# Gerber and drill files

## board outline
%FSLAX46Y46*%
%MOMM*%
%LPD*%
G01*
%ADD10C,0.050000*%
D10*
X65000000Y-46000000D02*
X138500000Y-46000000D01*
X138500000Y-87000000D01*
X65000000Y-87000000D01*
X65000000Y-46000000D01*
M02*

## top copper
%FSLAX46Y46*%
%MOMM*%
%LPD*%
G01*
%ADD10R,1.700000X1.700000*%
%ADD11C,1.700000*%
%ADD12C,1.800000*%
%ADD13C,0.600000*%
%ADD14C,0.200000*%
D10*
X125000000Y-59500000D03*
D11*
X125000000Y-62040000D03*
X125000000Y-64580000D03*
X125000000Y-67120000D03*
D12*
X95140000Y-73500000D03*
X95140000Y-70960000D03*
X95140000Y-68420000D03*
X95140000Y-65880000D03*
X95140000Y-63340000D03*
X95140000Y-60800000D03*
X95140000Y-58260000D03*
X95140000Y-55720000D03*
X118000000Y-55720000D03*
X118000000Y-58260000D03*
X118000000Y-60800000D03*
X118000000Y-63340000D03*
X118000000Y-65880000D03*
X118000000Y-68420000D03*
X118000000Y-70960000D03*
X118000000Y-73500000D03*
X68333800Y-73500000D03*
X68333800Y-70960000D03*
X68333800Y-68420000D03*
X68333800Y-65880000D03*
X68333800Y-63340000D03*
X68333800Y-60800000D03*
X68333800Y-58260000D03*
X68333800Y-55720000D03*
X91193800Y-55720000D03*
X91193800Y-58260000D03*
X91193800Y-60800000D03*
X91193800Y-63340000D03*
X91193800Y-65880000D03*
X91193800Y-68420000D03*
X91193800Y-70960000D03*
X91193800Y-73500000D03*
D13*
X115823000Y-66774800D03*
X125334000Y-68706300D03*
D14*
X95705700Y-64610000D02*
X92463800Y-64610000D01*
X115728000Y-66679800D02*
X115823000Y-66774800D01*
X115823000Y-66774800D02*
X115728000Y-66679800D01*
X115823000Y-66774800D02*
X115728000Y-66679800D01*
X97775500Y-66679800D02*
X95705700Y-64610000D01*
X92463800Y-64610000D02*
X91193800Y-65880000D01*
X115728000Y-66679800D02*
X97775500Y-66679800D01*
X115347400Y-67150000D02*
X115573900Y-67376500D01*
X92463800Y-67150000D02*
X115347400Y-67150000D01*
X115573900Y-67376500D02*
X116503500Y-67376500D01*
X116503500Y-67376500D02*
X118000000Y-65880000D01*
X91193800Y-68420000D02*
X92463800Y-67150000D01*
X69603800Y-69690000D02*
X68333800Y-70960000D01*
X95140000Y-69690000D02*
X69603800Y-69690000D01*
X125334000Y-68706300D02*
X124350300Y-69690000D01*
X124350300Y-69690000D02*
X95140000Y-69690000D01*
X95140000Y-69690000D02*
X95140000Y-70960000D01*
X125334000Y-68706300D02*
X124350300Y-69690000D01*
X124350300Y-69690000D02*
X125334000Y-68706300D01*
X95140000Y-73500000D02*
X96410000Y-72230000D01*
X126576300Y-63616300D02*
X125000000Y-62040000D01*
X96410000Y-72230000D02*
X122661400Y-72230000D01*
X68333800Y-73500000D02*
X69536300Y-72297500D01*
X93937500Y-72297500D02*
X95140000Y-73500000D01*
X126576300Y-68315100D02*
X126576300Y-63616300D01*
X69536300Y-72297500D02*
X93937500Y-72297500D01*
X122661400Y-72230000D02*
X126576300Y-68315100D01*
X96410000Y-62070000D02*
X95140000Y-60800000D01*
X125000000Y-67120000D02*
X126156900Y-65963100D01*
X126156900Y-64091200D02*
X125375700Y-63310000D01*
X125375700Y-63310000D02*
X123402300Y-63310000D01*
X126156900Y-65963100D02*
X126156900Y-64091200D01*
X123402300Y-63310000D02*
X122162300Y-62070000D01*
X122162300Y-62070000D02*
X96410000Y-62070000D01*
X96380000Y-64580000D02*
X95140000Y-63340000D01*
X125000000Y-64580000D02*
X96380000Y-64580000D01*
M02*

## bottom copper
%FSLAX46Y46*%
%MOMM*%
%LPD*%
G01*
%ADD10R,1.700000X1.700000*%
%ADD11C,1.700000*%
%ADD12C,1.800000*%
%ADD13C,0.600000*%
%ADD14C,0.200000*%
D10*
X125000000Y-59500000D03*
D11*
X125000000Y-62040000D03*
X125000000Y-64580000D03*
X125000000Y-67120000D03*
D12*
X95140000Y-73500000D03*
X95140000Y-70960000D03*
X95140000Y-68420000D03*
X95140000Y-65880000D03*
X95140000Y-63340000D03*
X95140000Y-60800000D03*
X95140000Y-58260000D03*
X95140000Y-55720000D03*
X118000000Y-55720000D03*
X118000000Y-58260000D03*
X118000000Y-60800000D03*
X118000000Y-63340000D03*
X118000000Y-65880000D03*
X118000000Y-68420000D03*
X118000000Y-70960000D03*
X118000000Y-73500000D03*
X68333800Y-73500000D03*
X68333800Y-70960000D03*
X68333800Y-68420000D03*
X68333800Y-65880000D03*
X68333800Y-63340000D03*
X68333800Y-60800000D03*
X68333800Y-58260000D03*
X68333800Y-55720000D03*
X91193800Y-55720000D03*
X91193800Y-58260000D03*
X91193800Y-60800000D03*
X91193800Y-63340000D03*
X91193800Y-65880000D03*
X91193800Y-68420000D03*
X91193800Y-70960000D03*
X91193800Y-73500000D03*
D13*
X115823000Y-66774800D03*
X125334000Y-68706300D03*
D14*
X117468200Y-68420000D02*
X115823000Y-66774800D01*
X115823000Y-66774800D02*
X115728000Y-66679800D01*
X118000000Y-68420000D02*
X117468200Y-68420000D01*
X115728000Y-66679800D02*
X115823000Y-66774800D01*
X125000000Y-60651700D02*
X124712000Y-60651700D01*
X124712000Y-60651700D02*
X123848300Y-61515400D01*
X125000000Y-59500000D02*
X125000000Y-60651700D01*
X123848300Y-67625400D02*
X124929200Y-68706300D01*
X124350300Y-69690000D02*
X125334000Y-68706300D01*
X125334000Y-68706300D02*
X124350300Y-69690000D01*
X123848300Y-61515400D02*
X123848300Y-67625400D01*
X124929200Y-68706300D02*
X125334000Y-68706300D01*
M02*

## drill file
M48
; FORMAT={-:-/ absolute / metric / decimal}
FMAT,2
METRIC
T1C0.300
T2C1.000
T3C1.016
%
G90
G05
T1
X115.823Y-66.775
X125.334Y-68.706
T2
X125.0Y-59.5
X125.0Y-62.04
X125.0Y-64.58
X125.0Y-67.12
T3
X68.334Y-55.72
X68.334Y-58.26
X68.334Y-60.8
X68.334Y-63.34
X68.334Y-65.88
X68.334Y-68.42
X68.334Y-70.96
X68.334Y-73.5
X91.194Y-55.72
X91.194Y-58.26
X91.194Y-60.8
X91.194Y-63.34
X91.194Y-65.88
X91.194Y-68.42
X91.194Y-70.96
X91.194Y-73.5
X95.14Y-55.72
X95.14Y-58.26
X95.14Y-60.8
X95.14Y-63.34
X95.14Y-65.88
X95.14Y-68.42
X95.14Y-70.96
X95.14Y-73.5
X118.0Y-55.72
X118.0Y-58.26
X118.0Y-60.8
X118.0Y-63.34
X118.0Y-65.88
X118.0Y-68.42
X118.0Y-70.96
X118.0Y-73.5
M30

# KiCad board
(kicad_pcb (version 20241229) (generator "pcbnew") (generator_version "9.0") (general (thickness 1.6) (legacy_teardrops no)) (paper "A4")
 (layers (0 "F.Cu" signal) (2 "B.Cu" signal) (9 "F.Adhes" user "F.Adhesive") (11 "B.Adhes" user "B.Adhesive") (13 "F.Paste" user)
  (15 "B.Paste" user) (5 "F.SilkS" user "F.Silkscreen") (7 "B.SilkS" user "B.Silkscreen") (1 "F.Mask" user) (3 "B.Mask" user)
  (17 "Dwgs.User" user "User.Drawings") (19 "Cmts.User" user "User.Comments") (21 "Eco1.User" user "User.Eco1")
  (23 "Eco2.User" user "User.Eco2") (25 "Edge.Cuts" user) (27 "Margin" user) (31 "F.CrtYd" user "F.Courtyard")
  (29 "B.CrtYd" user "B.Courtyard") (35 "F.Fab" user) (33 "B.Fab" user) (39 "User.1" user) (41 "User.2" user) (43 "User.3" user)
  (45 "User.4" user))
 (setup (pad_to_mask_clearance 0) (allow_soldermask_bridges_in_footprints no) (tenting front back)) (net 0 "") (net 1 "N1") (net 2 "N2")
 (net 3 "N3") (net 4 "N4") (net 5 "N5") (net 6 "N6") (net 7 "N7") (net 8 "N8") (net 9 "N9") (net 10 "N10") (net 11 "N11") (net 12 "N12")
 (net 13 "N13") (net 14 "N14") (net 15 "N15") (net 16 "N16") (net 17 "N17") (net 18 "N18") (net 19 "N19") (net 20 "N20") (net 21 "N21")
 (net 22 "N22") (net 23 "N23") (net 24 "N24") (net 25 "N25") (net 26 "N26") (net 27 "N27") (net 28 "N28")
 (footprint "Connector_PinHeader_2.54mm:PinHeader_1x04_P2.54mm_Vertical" (layer "F.Cu") (at 125 59.5)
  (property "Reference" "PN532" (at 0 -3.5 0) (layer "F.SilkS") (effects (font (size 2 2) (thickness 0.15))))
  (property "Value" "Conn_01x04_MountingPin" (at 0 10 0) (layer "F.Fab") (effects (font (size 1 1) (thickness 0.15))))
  (pad "1" thru_hole rect (at 0 0) (size 1.7 1.7) (drill 1) (layers "*.Cu" "*.Mask") (remove_unused_layers no) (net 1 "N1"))
  (pad "2" thru_hole circle (at 0 2.54) (size 1.7 1.7) (drill 1) (layers "*.Cu" "*.Mask") (remove_unused_layers no) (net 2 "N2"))
  (pad "3" thru_hole circle (at 0 5.08) (size 1.7 1.7) (drill 1) (layers "*.Cu" "*.Mask") (remove_unused_layers no) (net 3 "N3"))
  (pad "4" thru_hole circle (at 0 7.62) (size 1.7 1.7) (drill 1) (layers "*.Cu" "*.Mask") (remove_unused_layers no) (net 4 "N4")))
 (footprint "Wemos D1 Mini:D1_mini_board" (layer "F.Cu") (at 106.57 65.88)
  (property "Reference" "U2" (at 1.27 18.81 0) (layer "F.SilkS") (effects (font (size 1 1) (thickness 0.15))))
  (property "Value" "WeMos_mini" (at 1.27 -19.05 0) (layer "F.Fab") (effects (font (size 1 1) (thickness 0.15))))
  (pad "1" thru_hole circle (at -11.43 7.62) (size 1.8 1.8) (drill 1.016) (layers "*.Cu" "*.Mask" "F.SilkS") (remove_unused_layers no)
   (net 2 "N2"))
  (pad "2" thru_hole circle (at -11.43 5.08) (size 1.8 1.8) (drill 1.016) (layers "*.Cu" "*.Mask" "F.SilkS") (remove_unused_layers no)
   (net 1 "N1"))
  (pad "3" thru_hole circle (at -11.43 2.54) (size 1.8 1.8) (drill 1.016) (layers "*.Cu" "*.Mask" "F.SilkS") (remove_unused_layers no)
   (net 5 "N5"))
  (pad "4" thru_hole circle (at -11.43 0) (size 1.8 1.8) (drill 1.016) (layers "*.Cu" "*.Mask" "F.SilkS") (remove_unused_layers no)
   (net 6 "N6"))
  (pad "5" thru_hole circle (at -11.43 -2.54) (size 1.8 1.8) (drill 1.016) (layers "*.Cu" "*.Mask" "F.SilkS") (remove_unused_layers no)
   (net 3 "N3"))
  (pad "6" thru_hole circle (at -11.43 -5.08) (size 1.8 1.8) (drill 1.016) (layers "*.Cu" "*.Mask" "F.SilkS") (remove_unused_layers no)
   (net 4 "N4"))
  (pad "7" thru_hole circle (at -11.43 -7.62) (size 1.8 1.8) (drill 1.016) (layers "*.Cu" "*.Mask" "F.SilkS") (remove_unused_layers no)
   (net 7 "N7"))
  (pad "8" thru_hole circle (at -11.43 -10.16) (size 1.8 1.8) (drill 1.016) (layers "*.Cu" "*.Mask" "F.SilkS") (remove_unused_layers no)
   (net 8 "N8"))
  (pad "9" thru_hole circle (at 11.43 -10.16) (size 1.8 1.8) (drill 1.016) (layers "*.Cu" "*.Mask" "F.SilkS") (remove_unused_layers no)
   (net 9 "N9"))
  (pad "10" thru_hole circle (at 11.43 -7.62) (size 1.8 1.8) (drill 1.016) (layers "*.Cu" "*.Mask" "F.SilkS") (remove_unused_layers no)
   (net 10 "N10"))
  (pad "11" thru_hole circle (at 11.43 -5.08) (size 1.8 1.8) (drill 1.016) (layers "*.Cu" "*.Mask" "F.SilkS") (remove_unused_layers no)
   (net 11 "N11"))
  (pad "12" thru_hole circle (at 11.43 -2.54) (size 1.8 1.8) (drill 1.016) (layers "*.Cu" "*.Mask" "F.SilkS") (remove_unused_layers no)
   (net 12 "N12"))
  (pad "13" thru_hole circle (at 11.43 0) (size 1.8 1.8) (drill 1.016) (layers "*.Cu" "*.Mask" "F.SilkS") (remove_unused_layers no)
   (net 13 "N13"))
  (pad "14" thru_hole circle (at 11.43 2.54) (size 1.8 1.8) (drill 1.016) (layers "*.Cu" "*.Mask" "F.SilkS") (remove_unused_layers no)
   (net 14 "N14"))
  (pad "15" thru_hole circle (at 11.43 5.08) (size 1.8 1.8) (drill 1.016) (layers "*.Cu" "*.Mask" "F.SilkS") (remove_unused_layers no)
   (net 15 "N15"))
  (pad "16" thru_hole circle (at 11.43 7.62) (size 1.8 1.8) (drill 1.016) (layers "*.Cu" "*.Mask" "F.SilkS") (remove_unused_layers no)
   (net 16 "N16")))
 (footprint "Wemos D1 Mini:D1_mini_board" (layer "F.Cu") (at 79.7638 65.88)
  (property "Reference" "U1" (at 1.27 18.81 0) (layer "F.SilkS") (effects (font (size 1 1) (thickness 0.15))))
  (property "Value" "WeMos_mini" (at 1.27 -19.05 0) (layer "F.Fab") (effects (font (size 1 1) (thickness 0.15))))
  (pad "1" thru_hole circle (at -11.43 7.62) (size 1.8 1.8) (drill 1.016) (layers "*.Cu" "*.Mask" "F.SilkS") (remove_unused_layers no)
   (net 2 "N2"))
  (pad "2" thru_hole circle (at -11.43 5.08) (size 1.8 1.8) (drill 1.016) (layers "*.Cu" "*.Mask" "F.SilkS") (remove_unused_layers no)
   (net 1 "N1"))
  (pad "3" thru_hole circle (at -11.43 2.54) (size 1.8 1.8) (drill 1.016) (layers "*.Cu" "*.Mask" "F.SilkS") (remove_unused_layers no)
   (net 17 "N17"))
  (pad "4" thru_hole circle (at -11.43 0) (size 1.8 1.8) (drill 1.016) (layers "*.Cu" "*.Mask" "F.SilkS") (remove_unused_layers no)
   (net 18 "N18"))
  (pad "5" thru_hole circle (at -11.43 -2.54) (size 1.8 1.8) (drill 1.016) (layers "*.Cu" "*.Mask" "F.SilkS") (remove_unused_layers no)
   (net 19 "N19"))
  (pad "6" thru_hole circle (at -11.43 -5.08) (size 1.8 1.8) (drill 1.016) (layers "*.Cu" "*.Mask" "F.SilkS") (remove_unused_layers no)
   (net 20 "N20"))
  (pad "7" thru_hole circle (at -11.43 -7.62) (size 1.8 1.8) (drill 1.016) (layers "*.Cu" "*.Mask" "F.SilkS") (remove_unused_layers no)
   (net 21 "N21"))
  (pad "8" thru_hole circle (at -11.43 -10.16) (size 1.8 1.8) (drill 1.016) (layers "*.Cu" "*.Mask" "F.SilkS") (remove_unused_layers no)
   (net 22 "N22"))
  (pad "9" thru_hole circle (at 11.43 -10.16) (size 1.8 1.8) (drill 1.016) (layers "*.Cu" "*.Mask" "F.SilkS") (remove_unused_layers no)
   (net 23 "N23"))
  (pad "10" thru_hole circle (at 11.43 -7.62) (size 1.8 1.8) (drill 1.016) (layers "*.Cu" "*.Mask" "F.SilkS") (remove_unused_layers no)
   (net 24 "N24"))
  (pad "11" thru_hole circle (at 11.43 -5.08) (size 1.8 1.8) (drill 1.016) (layers "*.Cu" "*.Mask" "F.SilkS") (remove_unused_layers no)
   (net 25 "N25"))
  (pad "12" thru_hole circle (at 11.43 -2.54) (size 1.8 1.8) (drill 1.016) (layers "*.Cu" "*.Mask" "F.SilkS") (remove_unused_layers no)
   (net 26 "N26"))
  (pad "13" thru_hole circle (at 11.43 0) (size 1.8 1.8) (drill 1.016) (layers "*.Cu" "*.Mask" "F.SilkS") (remove_unused_layers no)
   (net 14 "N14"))
  (pad "14" thru_hole circle (at 11.43 2.54) (size 1.8 1.8) (drill 1.016) (layers "*.Cu" "*.Mask" "F.SilkS") (remove_unused_layers no)
   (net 13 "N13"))
  (pad "15" thru_hole circle (at 11.43 5.08) (size 1.8 1.8) (drill 1.016) (layers "*.Cu" "*.Mask" "F.SilkS") (remove_unused_layers no)
   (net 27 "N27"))
  (pad "16" thru_hole circle (at 11.43 7.62) (size 1.8 1.8) (drill 1.016) (layers "*.Cu" "*.Mask" "F.SilkS") (remove_unused_layers no)
   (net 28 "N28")))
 (gr_rect (start 65 46) (end 138.5 87) (stroke (width 0.05) (type default)) (fill no) (layer "Edge.Cuts"))
 (segment (start 95.7057 64.61) (end 92.4638 64.61) (width 0.2) (layer "F.Cu") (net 14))
 (segment (start 115.728 66.6798) (end 115.823 66.7748) (width 0.2) (layer "F.Cu") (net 14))
 (segment (start 115.823 66.7748) (end 115.728 66.6798) (width 0.2) (layer "F.Cu") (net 14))
 (segment (start 115.823 66.7748) (end 115.728 66.6798) (width 0.2) (layer "F.Cu") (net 14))
 (segment (start 97.7755 66.6798) (end 95.7057 64.61) (width 0.2) (layer "F.Cu") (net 14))
 (segment (start 92.4638 64.61) (end 91.1938 65.88) (width 0.2) (layer "F.Cu") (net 14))
 (segment (start 115.728 66.6798) (end 97.7755 66.6798) (width 0.2) (layer "F.Cu") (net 14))
 (via (at 115.823 66.7748) (size 0.6) (drill 0.3) (layers "F.Cu" "B.Cu") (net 14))
 (segment (start 117.4682 68.42) (end 115.823 66.7748) (width 0.2) (layer "B.Cu") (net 14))
 (segment (start 115.823 66.7748) (end 115.728 66.6798) (width 0.2) (layer "B.Cu") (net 14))
 (segment (start 118 68.42) (end 117.4682 68.42) (width 0.2) (layer "B.Cu") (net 14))
 (segment (start 115.728 66.6798) (end 115.823 66.7748) (width 0.2) (layer "B.Cu") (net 14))
 (segment (start 115.3474 67.15) (end 115.5739 67.3765) (width 0.2) (layer "F.Cu") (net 13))
 (segment (start 92.4638 67.15) (end 115.3474 67.15) (width 0.2) (layer "F.Cu") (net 13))
 (segment (start 115.5739 67.3765) (end 116.5035 67.3765) (width 0.2) (layer "F.Cu") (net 13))
 (segment (start 116.5035 67.3765) (end 118 65.88) (width 0.2) (layer "F.Cu") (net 13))
 (segment (start 91.1938 68.42) (end 92.4638 67.15) (width 0.2) (layer "F.Cu") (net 13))
 (segment (start 69.6038 69.69) (end 68.3338 70.96) (width 0.2) (layer "F.Cu") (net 1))
 (segment (start 95.14 69.69) (end 69.6038 69.69) (width 0.2) (layer "F.Cu") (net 1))
 (segment (start 125.334 68.7063) (end 124.3503 69.69) (width 0.2) (layer "F.Cu") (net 1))
 (segment (start 124.3503 69.69) (end 95.14 69.69) (width 0.2) (layer "F.Cu") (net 1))
 (segment (start 95.14 69.69) (end 95.14 70.96) (width 0.2) (layer "F.Cu") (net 1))
 (segment (start 125.334 68.7063) (end 124.3503 69.69) (width 0.2) (layer "F.Cu") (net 1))
 (segment (start 124.3503 69.69) (end 125.334 68.7063) (width 0.2) (layer "F.Cu") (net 1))
 (via (at 125.334 68.7063) (size 0.6) (drill 0.3) (layers "F.Cu" "B.Cu") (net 1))
 (segment (start 125 60.6517) (end 124.712 60.6517) (width 0.2) (layer "B.Cu") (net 1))
 (segment (start 124.712 60.6517) (end 123.8483 61.5154) (width 0.2) (layer "B.Cu") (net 1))
 (segment (start 125 59.5) (end 125 60.6517) (width 0.2) (layer "B.Cu") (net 1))
 (segment (start 123.8483 67.6254) (end 124.9292 68.7063) (width 0.2) (layer "B.Cu") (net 1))
 (segment (start 124.3503 69.69) (end 125.334 68.7063) (width 0.2) (layer "B.Cu") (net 1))
 (segment (start 125.334 68.7063) (end 124.3503 69.69) (width 0.2) (layer "B.Cu") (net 1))
 (segment (start 123.8483 61.5154) (end 123.8483 67.6254) (width 0.2) (layer "B.Cu") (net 1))
 (segment (start 124.9292 68.7063) (end 125.334 68.7063) (width 0.2) (layer "B.Cu") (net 1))
 (segment (start 95.14 73.5) (end 96.41 72.23) (width 0.2) (layer "F.Cu") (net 2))
 (segment (start 126.5763 63.6163) (end 125 62.04) (width 0.2) (layer "F.Cu") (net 2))
 (segment (start 96.41 72.23) (end 122.6614 72.23) (width 0.2) (layer "F.Cu") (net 2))
 (segment (start 68.3338 73.5) (end 69.5363 72.2975) (width 0.2) (layer "F.Cu") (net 2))
 (segment (start 93.9375 72.2975) (end 95.14 73.5) (width 0.2) (layer "F.Cu") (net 2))
 (segment (start 126.5763 68.3151) (end 126.5763 63.6163) (width 0.2) (layer "F.Cu") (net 2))
 (segment (start 69.5363 72.2975) (end 93.9375 72.2975) (width 0.2) (layer "F.Cu") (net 2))
 (segment (start 122.6614 72.23) (end 126.5763 68.3151) (width 0.2) (layer "F.Cu") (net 2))
 (segment (start 96.41 62.07) (end 95.14 60.8) (width 0.2) (layer "F.Cu") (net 4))
 (segment (start 125 67.12) (end 126.1569 65.9631) (width 0.2) (layer "F.Cu") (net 4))
 (segment (start 126.1569 64.0912) (end 125.3757 63.31) (width 0.2) (layer "F.Cu") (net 4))
 (segment (start 125.3757 63.31) (end 123.4023 63.31) (width 0.2) (layer "F.Cu") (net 4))
 (segment (start 126.1569 65.9631) (end 126.1569 64.0912) (width 0.2) (layer "F.Cu") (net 4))
 (segment (start 123.4023 63.31) (end 122.1623 62.07) (width 0.2) (layer "F.Cu") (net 4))
 (segment (start 122.1623 62.07) (end 96.41 62.07) (width 0.2) (layer "F.Cu") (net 4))
 (segment (start 96.38 64.58) (end 95.14 63.34) (width 0.2) (layer "F.Cu") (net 3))
 (segment (start 125 64.58) (end 96.38 64.58) (width 0.2) (layer "F.Cu") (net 3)))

